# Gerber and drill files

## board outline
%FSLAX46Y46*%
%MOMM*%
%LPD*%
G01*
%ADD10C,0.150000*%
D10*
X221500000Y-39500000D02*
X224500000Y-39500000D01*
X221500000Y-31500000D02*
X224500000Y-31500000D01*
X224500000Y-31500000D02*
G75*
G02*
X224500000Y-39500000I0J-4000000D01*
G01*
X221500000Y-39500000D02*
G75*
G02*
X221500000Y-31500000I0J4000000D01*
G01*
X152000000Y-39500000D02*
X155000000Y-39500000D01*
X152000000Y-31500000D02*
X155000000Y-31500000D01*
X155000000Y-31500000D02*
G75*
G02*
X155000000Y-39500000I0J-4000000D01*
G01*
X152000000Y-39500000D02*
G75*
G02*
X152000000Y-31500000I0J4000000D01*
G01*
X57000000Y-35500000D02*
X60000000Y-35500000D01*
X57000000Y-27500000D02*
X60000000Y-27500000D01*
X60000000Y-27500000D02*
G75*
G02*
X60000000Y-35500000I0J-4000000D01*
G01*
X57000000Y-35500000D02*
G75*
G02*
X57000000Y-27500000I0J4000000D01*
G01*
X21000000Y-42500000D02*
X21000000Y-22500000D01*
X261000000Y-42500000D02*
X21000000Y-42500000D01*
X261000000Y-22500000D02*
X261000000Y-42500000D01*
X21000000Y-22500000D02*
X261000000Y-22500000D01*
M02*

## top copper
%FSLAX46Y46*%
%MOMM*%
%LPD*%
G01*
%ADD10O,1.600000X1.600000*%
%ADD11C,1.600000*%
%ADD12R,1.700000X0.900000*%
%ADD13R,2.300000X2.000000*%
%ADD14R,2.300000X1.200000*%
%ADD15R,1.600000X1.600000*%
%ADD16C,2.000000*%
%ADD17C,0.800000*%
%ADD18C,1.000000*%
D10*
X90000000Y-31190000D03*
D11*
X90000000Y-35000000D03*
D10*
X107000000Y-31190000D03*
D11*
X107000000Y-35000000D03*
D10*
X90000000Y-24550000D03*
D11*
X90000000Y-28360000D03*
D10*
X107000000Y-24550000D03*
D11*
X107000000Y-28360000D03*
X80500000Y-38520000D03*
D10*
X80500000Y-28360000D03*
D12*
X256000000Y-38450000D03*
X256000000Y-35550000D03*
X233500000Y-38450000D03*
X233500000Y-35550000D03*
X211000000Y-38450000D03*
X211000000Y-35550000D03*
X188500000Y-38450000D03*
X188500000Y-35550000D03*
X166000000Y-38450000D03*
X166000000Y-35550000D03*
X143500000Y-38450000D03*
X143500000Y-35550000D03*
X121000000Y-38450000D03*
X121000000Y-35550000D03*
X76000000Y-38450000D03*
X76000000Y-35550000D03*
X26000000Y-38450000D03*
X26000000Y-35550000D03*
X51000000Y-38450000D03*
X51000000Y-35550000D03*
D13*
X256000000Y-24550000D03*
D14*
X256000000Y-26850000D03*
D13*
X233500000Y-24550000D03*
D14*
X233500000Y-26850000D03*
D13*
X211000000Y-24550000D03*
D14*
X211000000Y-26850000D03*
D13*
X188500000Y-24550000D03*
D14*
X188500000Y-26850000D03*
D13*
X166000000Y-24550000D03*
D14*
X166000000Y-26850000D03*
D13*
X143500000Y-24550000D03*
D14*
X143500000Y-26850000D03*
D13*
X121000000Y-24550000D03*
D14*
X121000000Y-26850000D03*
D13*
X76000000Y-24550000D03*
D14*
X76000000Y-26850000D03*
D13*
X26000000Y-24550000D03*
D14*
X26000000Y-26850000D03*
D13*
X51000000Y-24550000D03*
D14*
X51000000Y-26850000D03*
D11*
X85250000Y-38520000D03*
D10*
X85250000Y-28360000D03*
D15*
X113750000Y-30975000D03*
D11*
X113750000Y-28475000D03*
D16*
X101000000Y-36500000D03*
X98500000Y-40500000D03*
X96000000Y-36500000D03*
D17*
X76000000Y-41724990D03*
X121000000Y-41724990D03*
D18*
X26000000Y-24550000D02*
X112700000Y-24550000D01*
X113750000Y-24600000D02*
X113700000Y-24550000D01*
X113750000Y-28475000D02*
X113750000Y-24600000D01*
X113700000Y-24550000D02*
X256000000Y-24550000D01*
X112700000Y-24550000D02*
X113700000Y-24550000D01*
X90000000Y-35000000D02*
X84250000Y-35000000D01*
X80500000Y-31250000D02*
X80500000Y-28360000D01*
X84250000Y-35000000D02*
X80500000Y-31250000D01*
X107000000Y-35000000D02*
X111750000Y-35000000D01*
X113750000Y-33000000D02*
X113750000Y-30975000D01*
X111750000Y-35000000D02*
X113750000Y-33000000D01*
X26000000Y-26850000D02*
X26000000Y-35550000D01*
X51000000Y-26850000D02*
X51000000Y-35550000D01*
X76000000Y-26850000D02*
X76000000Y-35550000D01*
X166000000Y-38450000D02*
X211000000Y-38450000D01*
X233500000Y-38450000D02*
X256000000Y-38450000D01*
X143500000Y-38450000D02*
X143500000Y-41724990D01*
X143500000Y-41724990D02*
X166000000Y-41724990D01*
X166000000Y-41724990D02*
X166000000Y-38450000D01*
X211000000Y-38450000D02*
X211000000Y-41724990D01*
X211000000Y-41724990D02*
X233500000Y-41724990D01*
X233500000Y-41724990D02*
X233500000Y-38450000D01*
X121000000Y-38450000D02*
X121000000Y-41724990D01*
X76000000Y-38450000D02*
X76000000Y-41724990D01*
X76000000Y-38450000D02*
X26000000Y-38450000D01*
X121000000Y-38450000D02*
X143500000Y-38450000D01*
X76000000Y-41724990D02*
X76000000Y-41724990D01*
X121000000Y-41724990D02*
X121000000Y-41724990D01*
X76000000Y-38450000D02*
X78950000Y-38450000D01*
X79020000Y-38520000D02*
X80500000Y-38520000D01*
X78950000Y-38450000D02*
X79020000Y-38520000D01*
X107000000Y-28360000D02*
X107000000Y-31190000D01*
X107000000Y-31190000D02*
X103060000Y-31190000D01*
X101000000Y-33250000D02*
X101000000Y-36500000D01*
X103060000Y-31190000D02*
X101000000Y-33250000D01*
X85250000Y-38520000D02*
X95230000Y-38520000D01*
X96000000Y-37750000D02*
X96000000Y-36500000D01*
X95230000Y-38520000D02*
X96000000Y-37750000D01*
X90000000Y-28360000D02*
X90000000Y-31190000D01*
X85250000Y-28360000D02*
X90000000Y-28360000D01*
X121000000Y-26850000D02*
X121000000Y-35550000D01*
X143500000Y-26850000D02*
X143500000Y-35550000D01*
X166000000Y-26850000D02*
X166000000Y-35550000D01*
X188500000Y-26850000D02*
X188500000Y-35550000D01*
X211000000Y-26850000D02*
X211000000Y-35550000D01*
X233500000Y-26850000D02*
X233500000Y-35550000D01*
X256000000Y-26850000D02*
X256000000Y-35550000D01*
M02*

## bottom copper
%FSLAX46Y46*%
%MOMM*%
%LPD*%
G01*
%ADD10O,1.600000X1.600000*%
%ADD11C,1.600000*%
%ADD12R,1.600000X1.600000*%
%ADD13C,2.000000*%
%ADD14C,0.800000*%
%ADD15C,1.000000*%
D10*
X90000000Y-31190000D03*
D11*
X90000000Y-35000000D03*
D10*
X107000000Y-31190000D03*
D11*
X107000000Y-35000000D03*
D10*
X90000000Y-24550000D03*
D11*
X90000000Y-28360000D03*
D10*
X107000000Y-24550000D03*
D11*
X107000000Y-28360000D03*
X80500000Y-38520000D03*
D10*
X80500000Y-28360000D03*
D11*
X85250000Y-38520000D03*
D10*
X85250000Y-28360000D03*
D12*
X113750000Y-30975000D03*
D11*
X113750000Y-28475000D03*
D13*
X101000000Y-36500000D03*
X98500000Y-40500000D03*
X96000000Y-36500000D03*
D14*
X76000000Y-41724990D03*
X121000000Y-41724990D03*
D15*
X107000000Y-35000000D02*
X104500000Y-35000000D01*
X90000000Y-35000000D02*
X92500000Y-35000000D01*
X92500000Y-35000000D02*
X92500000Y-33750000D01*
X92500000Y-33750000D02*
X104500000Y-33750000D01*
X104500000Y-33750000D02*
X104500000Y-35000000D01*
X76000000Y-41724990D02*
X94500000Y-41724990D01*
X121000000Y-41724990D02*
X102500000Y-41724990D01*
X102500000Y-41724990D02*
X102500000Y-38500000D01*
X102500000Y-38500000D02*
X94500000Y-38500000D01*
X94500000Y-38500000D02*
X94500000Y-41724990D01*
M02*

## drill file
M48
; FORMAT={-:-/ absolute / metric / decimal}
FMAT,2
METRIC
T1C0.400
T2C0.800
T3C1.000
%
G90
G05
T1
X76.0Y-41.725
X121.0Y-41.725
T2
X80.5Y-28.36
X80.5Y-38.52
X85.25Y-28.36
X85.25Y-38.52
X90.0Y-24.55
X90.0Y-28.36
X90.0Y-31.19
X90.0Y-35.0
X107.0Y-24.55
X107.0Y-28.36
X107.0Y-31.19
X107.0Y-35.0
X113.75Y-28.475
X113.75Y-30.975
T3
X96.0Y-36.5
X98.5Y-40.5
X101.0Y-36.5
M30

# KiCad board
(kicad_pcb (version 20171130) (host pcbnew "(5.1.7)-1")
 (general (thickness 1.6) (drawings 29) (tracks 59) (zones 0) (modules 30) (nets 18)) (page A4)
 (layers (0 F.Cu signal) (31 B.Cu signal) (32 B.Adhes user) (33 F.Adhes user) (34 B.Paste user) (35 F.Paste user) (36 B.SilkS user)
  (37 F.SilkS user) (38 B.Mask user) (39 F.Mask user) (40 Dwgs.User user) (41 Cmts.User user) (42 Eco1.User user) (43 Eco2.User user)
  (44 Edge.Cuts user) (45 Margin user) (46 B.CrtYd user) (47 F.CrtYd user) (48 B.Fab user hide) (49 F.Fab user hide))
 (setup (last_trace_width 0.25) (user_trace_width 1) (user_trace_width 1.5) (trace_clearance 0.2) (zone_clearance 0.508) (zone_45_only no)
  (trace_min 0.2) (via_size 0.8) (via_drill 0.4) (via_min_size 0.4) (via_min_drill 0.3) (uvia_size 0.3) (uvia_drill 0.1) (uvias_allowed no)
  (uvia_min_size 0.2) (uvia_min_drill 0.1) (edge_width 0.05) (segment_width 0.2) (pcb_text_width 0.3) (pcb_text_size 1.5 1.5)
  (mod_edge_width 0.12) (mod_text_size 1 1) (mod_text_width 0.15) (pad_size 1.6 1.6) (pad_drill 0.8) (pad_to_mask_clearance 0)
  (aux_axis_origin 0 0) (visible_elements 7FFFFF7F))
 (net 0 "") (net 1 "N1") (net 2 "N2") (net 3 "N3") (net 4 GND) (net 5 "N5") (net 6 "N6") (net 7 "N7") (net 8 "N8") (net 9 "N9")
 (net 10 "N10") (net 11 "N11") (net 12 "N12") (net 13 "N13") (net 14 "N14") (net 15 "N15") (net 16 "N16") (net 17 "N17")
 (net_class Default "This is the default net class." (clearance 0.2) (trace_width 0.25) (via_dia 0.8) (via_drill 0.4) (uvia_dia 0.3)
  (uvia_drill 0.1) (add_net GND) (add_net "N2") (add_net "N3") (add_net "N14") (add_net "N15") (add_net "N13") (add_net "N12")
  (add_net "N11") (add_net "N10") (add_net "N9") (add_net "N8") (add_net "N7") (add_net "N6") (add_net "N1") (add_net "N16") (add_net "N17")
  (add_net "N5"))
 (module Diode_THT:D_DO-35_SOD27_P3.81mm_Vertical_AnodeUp (layer F.Cu) (at 90 35 90)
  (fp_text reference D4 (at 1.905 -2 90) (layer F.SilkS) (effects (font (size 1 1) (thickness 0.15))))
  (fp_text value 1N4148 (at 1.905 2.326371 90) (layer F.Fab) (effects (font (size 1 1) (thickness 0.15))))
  (pad 2 thru_hole oval (at 3.81 0 90) (size 1.6 1.6) (drill 0.8) (layers *.Cu *.Mask) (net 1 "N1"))
  (pad 1 thru_hole circle (at 0 0 90) (size 1.6 1.6) (drill 0.8) (layers *.Cu *.Mask) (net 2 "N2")))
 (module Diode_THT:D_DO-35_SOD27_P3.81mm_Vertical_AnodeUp (layer F.Cu) (at 107 35 90)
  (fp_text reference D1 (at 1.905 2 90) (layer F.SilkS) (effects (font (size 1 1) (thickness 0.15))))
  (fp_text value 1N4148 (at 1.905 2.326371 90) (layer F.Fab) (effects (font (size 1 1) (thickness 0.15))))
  (pad 2 thru_hole oval (at 3.81 0 90) (size 1.6 1.6) (drill 0.8) (layers *.Cu *.Mask) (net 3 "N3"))
  (pad 1 thru_hole circle (at 0 0 90) (size 1.6 1.6) (drill 0.8) (layers *.Cu *.Mask) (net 2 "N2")))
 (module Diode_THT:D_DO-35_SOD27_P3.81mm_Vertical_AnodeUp (layer F.Cu) (at 90 28.36 90)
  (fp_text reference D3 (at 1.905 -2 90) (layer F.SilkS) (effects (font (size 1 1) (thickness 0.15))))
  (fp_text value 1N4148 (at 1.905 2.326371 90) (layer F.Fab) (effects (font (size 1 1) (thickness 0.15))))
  (pad 2 thru_hole oval (at 3.81 0 90) (size 1.6 1.6) (drill 0.8) (layers *.Cu *.Mask) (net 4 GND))
  (pad 1 thru_hole circle (at 0 0 90) (size 1.6 1.6) (drill 0.8) (layers *.Cu *.Mask) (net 1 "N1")))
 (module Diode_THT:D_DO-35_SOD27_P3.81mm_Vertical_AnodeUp (layer F.Cu) (at 107 28.36 90)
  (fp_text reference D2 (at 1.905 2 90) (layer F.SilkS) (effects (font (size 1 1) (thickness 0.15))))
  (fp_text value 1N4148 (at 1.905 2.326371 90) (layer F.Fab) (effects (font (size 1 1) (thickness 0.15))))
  (pad 2 thru_hole oval (at 3.81 0 90) (size 1.6 1.6) (drill 0.8) (layers *.Cu *.Mask) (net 4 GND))
  (pad 1 thru_hole circle (at 0 0 90) (size 1.6 1.6) (drill 0.8) (layers *.Cu *.Mask) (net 3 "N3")))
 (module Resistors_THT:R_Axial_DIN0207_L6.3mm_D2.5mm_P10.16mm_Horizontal (layer F.Cu) (at 80.5 38.52 90)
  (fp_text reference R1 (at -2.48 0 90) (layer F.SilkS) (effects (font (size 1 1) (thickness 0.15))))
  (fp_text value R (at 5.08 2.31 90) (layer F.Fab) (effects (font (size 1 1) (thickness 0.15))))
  (pad 1 thru_hole circle (at 0 0 90) (size 1.6 1.6) (drill 0.8) (layers *.Cu *.Mask) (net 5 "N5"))
  (pad 2 thru_hole oval (at 10.16 0 90) (size 1.6 1.6) (drill 0.8) (layers *.Cu *.Mask) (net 2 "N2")))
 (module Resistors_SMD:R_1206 (layer F.Cu) (at 256 37 90)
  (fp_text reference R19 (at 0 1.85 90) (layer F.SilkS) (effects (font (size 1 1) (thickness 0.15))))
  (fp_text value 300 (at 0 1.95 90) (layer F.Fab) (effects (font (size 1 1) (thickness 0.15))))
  (pad 1 smd rect (at -1.45 0 90) (size 0.9 1.7) (layers F.Cu F.Paste F.Mask) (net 5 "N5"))
  (pad 2 smd rect (at 1.45 0 90) (size 0.9 1.7) (layers F.Cu F.Paste F.Mask) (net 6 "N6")))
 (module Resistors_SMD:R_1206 (layer F.Cu) (at 233.5 37 90)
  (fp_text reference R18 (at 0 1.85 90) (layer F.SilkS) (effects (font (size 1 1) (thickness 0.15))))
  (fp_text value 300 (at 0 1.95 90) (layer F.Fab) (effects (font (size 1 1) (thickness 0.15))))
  (pad 1 smd rect (at -1.45 0 90) (size 0.9 1.7) (layers F.Cu F.Paste F.Mask) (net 5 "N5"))
  (pad 2 smd rect (at 1.45 0 90) (size 0.9 1.7) (layers F.Cu F.Paste F.Mask) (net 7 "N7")))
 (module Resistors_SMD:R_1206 (layer F.Cu) (at 211 37 90)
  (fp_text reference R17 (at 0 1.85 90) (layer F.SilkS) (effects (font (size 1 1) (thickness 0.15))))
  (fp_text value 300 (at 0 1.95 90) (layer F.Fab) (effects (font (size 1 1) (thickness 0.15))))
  (pad 1 smd rect (at -1.45 0 90) (size 0.9 1.7) (layers F.Cu F.Paste F.Mask) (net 5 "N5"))
  (pad 2 smd rect (at 1.45 0 90) (size 0.9 1.7) (layers F.Cu F.Paste F.Mask) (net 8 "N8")))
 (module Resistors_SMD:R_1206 (layer F.Cu) (at 188.5 37 90)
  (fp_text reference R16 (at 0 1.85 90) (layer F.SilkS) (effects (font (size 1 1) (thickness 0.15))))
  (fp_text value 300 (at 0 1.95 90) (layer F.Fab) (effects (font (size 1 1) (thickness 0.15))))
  (pad 1 smd rect (at -1.45 0 90) (size 0.9 1.7) (layers F.Cu F.Paste F.Mask) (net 5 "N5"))
  (pad 2 smd rect (at 1.45 0 90) (size 0.9 1.7) (layers F.Cu F.Paste F.Mask) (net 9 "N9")))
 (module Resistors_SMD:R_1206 (layer F.Cu) (at 166 37 90)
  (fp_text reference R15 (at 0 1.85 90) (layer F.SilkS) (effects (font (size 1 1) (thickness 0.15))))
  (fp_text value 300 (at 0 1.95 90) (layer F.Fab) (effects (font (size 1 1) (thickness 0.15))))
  (pad 1 smd rect (at -1.45 0 90) (size 0.9 1.7) (layers F.Cu F.Paste F.Mask) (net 5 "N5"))
  (pad 2 smd rect (at 1.45 0 90) (size 0.9 1.7) (layers F.Cu F.Paste F.Mask) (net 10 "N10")))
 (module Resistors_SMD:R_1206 (layer F.Cu) (at 143.5 37 90)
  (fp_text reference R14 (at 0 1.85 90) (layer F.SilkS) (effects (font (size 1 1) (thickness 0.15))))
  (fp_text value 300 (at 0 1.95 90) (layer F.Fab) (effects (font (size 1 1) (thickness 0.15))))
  (pad 1 smd rect (at -1.45 0 90) (size 0.9 1.7) (layers F.Cu F.Paste F.Mask) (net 5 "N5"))
  (pad 2 smd rect (at 1.45 0 90) (size 0.9 1.7) (layers F.Cu F.Paste F.Mask) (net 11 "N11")))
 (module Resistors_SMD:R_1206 (layer F.Cu) (at 121 37 90)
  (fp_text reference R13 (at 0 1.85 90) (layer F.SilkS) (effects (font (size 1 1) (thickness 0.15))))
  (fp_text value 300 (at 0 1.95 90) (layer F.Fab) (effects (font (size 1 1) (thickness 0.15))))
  (pad 1 smd rect (at -1.45 0 90) (size 0.9 1.7) (layers F.Cu F.Paste F.Mask) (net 5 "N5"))
  (pad 2 smd rect (at 1.45 0 90) (size 0.9 1.7) (layers F.Cu F.Paste F.Mask) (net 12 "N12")))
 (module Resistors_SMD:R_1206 (layer F.Cu) (at 76 37 90)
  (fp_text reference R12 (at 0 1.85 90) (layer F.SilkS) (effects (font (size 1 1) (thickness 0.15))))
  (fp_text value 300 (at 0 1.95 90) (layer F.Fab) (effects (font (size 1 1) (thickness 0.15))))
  (pad 1 smd rect (at -1.45 0 90) (size 0.9 1.7) (layers F.Cu F.Paste F.Mask) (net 5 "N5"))
  (pad 2 smd rect (at 1.45 0 90) (size 0.9 1.7) (layers F.Cu F.Paste F.Mask) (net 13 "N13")))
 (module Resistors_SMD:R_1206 (layer F.Cu) (at 26 37 90)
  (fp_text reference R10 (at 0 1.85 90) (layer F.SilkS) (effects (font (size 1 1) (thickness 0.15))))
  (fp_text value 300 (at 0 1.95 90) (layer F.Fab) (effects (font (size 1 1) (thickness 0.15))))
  (pad 1 smd rect (at -1.45 0 90) (size 0.9 1.7) (layers F.Cu F.Paste F.Mask) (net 5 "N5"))
  (pad 2 smd rect (at 1.45 0 90) (size 0.9 1.7) (layers F.Cu F.Paste F.Mask) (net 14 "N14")))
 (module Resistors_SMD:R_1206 (layer F.Cu) (at 51 37 90)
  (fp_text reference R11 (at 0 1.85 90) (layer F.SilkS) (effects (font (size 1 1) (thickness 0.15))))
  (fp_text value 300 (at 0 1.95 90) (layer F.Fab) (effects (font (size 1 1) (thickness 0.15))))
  (pad 1 smd rect (at -1.45 0 90) (size 0.9 1.7) (layers F.Cu F.Paste F.Mask) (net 5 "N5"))
  (pad 2 smd rect (at 1.45 0 90) (size 0.9 1.7) (layers F.Cu F.Paste F.Mask) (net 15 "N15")))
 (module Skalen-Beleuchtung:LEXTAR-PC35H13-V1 (layer F.Cu) (at 256 25.5 90)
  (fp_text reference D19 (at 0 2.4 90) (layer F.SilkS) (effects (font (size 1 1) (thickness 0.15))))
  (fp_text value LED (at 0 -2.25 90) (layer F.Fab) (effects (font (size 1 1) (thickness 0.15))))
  (pad 1 smd rect (at 0.95 0 90) (size 2 2.3) (layers F.Cu F.Paste F.Mask) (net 4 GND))
  (pad 2 smd rect (at -1.35 0 90) (size 1.2 2.3) (layers F.Cu F.Paste F.Mask) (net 6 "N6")))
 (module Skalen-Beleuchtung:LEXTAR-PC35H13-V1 (layer F.Cu) (at 233.5 25.5 90)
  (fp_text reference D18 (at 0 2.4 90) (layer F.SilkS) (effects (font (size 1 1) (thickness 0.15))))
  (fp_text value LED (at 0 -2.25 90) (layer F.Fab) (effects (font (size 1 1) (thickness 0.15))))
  (pad 1 smd rect (at 0.95 0 90) (size 2 2.3) (layers F.Cu F.Paste F.Mask) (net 4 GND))
  (pad 2 smd rect (at -1.35 0 90) (size 1.2 2.3) (layers F.Cu F.Paste F.Mask) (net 7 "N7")))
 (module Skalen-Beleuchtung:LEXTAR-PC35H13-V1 (layer F.Cu) (at 211 25.5 90)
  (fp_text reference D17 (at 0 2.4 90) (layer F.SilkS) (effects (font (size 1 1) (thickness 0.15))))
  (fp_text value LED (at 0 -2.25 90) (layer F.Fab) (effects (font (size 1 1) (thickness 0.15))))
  (pad 1 smd rect (at 0.95 0 90) (size 2 2.3) (layers F.Cu F.Paste F.Mask) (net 4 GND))
  (pad 2 smd rect (at -1.35 0 90) (size 1.2 2.3) (layers F.Cu F.Paste F.Mask) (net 8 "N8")))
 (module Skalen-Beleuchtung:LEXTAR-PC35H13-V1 (layer F.Cu) (at 188.5 25.5 90)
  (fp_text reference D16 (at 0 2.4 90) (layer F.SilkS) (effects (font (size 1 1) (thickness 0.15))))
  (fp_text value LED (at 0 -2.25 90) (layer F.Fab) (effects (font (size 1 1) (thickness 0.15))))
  (pad 1 smd rect (at 0.95 0 90) (size 2 2.3) (layers F.Cu F.Paste F.Mask) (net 4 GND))
  (pad 2 smd rect (at -1.35 0 90) (size 1.2 2.3) (layers F.Cu F.Paste F.Mask) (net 9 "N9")))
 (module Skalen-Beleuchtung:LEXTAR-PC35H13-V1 (layer F.Cu) (at 166 25.5 90)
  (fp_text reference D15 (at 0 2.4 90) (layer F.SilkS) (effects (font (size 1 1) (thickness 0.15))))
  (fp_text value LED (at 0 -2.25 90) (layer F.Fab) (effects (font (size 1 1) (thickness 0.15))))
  (pad 1 smd rect (at 0.95 0 90) (size 2 2.3) (layers F.Cu F.Paste F.Mask) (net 4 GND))
  (pad 2 smd rect (at -1.35 0 90) (size 1.2 2.3) (layers F.Cu F.Paste F.Mask) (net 10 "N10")))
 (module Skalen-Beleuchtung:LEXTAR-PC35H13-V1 (layer F.Cu) (at 143.5 25.5 90)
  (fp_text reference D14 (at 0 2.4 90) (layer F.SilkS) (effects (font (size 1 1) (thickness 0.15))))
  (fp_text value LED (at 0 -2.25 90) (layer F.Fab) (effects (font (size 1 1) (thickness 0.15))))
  (pad 1 smd rect (at 0.95 0 90) (size 2 2.3) (layers F.Cu F.Paste F.Mask) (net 4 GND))
  (pad 2 smd rect (at -1.35 0 90) (size 1.2 2.3) (layers F.Cu F.Paste F.Mask) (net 11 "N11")))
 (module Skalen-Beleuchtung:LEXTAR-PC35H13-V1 (layer F.Cu) (at 121 25.5 90)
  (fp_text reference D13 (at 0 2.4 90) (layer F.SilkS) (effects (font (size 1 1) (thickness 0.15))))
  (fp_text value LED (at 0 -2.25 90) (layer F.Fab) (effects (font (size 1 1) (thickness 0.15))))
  (pad 1 smd rect (at 0.95 0 90) (size 2 2.3) (layers F.Cu F.Paste F.Mask) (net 4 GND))
  (pad 2 smd rect (at -1.35 0 90) (size 1.2 2.3) (layers F.Cu F.Paste F.Mask) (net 12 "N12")))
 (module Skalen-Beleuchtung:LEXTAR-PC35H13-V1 (layer F.Cu) (at 76 25.5 90)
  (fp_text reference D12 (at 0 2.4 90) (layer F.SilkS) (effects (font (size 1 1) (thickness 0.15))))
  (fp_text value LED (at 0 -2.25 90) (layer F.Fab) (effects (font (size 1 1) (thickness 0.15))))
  (pad 1 smd rect (at 0.95 0 90) (size 2 2.3) (layers F.Cu F.Paste F.Mask) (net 4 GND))
  (pad 2 smd rect (at -1.35 0 90) (size 1.2 2.3) (layers F.Cu F.Paste F.Mask) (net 13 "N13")))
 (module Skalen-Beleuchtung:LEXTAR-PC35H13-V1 (layer F.Cu) (at 26 25.5 90)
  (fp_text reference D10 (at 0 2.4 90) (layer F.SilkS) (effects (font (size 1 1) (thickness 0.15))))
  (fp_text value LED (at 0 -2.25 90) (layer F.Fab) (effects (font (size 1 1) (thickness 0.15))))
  (pad 1 smd rect (at 0.95 0 90) (size 2 2.3) (layers F.Cu F.Paste F.Mask) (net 4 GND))
  (pad 2 smd rect (at -1.35 0 90) (size 1.2 2.3) (layers F.Cu F.Paste F.Mask) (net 14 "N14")))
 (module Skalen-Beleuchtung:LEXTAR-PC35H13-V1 (layer F.Cu) (at 51 25.5 90)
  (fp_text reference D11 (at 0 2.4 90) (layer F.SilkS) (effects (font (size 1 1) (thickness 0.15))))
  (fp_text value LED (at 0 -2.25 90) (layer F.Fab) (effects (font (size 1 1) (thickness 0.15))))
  (pad 1 smd rect (at 0.95 0 90) (size 2 2.3) (layers F.Cu F.Paste F.Mask) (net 4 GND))
  (pad 2 smd rect (at -1.35 0 90) (size 1.2 2.3) (layers F.Cu F.Paste F.Mask) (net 15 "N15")))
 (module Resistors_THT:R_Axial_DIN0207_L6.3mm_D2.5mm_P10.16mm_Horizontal (layer F.Cu) (at 85.25 38.52 90)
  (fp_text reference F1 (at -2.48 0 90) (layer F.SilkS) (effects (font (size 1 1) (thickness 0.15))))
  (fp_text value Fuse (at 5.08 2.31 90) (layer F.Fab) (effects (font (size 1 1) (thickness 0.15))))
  (pad 1 thru_hole circle (at 0 0 90) (size 1.6 1.6) (drill 0.8) (layers *.Cu *.Mask) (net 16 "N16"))
  (pad 2 thru_hole oval (at 10.16 0 90) (size 1.6 1.6) (drill 0.8) (layers *.Cu *.Mask) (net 1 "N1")))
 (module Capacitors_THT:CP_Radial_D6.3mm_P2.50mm (layer F.Cu) (at 113.75 30.975 90)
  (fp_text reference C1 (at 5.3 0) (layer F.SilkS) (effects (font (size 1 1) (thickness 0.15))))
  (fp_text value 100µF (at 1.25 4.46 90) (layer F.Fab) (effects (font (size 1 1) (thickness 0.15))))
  (pad 1 thru_hole rect (at 0 0 90) (size 1.6 1.6) (drill 0.8) (layers *.Cu *.Mask) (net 2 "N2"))
  (pad 2 thru_hole circle (at 2.5 0 90) (size 1.6 1.6) (drill 0.8) (layers *.Cu *.Mask) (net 4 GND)))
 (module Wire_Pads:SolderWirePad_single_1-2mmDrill (layer F.Cu) (at 101 36.5)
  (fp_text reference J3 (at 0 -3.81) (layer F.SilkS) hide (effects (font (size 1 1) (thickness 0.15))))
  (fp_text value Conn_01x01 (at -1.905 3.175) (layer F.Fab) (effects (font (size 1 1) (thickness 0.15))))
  (pad 1 thru_hole circle (at 0 0) (size 2 2) (drill 1) (layers *.Cu *.Mask) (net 3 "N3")))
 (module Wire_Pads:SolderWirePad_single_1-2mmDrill (layer F.Cu) (at 98.5 40.5)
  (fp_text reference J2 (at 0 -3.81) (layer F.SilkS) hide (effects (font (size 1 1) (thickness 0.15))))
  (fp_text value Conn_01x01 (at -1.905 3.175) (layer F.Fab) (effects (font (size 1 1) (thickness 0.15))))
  (pad 1 thru_hole circle (at 0 0) (size 2 2) (drill 1) (layers *.Cu *.Mask) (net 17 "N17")))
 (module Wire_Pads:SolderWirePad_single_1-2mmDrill (layer F.Cu) (at 96 36.5)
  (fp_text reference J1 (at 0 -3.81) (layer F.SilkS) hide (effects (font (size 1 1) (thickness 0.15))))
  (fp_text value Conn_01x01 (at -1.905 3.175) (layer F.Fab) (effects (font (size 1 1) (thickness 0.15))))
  (pad 1 thru_hole circle (at 0 0) (size 2 2) (drill 1) (layers *.Cu *.Mask) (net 16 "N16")))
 (gr_line (start 221.5 39.5) (end 224.5 39.5) (layer Edge.Cuts) (width 0.15))
 (gr_line (start 221.5 31.5) (end 224.5 31.5) (layer Edge.Cuts) (width 0.15))
 (gr_arc (start 224.5 35.5) (end 224.5 39.5) (angle -180) (layer Edge.Cuts) (width 0.15))
 (gr_arc (start 221.5 35.5) (end 221.5 31.5) (angle -180) (layer Edge.Cuts) (width 0.15))
 (gr_line (start 152 39.5) (end 155 39.5) (layer Edge.Cuts) (width 0.15))
 (gr_line (start 152 31.5) (end 155 31.5) (layer Edge.Cuts) (width 0.15))
 (gr_arc (start 155 35.5) (end 155 39.5) (angle -180) (layer Edge.Cuts) (width 0.15))
 (gr_arc (start 152 35.5) (end 152 31.5) (angle -180) (layer Edge.Cuts) (width 0.15))
 (gr_line (start 57 35.5) (end 60 35.5) (layer Edge.Cuts) (width 0.15))
 (gr_line (start 57 27.5) (end 60 27.5) (layer Edge.Cuts) (width 0.15))
 (gr_arc (start 60 31.5) (end 60 35.5) (angle -180) (layer Edge.Cuts) (width 0.15))
 (gr_arc (start 57 31.5) (end 57 27.5) (angle -180) (layer Edge.Cuts) (width 0.15))
 (gr_line (start 21 42.5) (end 21 22.5) (layer Edge.Cuts) (width 0.15))
 (gr_line (start 261 42.5) (end 21 42.5) (layer Edge.Cuts) (width 0.15))
 (gr_line (start 261 22.5) (end 261 42.5) (layer Edge.Cuts) (width 0.15))
 (gr_line (start 21 22.5) (end 261 22.5) (layer Edge.Cuts) (width 0.15))
 (segment (start 26 24.55) (end 112.7 24.55) (width 1) (layer F.Cu) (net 4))
 (segment (start 113.75 24.6) (end 113.7 24.55) (width 1) (layer F.Cu) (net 4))
 (segment (start 113.75 28.475) (end 113.75 24.6) (width 1) (layer F.Cu) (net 4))
 (segment (start 113.7 24.55) (end 256 24.55) (width 1) (layer F.Cu) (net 4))
 (segment (start 112.7 24.55) (end 113.7 24.55) (width 1) (layer F.Cu) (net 4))
 (segment (start 107 35) (end 104.5 35) (width 1) (layer B.Cu) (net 2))
 (segment (start 90 35) (end 92.5 35) (width 1) (layer B.Cu) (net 2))
 (segment (start 92.5 35) (end 92.5 33.75) (width 1) (layer B.Cu) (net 2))
 (segment (start 92.5 33.75) (end 104.5 33.75) (width 1) (layer B.Cu) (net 2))
 (segment (start 104.5 33.75) (end 104.5 35) (width 1) (layer B.Cu) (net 2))
 (segment (start 90 35) (end 84.25 35) (width 1) (layer F.Cu) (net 2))
 (segment (start 80.5 31.25) (end 80.5 28.36) (width 1) (layer F.Cu) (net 2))
 (segment (start 84.25 35) (end 80.5 31.25) (width 1) (layer F.Cu) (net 2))
 (segment (start 107 35) (end 111.75 35) (width 1) (layer F.Cu) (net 2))
 (segment (start 113.75 33) (end 113.75 30.975) (width 1) (layer F.Cu) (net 2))
 (segment (start 111.75 35) (end 113.75 33) (width 1) (layer F.Cu) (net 2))
 (segment (start 26 26.85) (end 26 35.55) (width 1) (layer F.Cu) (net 14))
 (segment (start 51 26.85) (end 51 35.55) (width 1) (layer F.Cu) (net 15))
 (segment (start 76 26.85) (end 76 35.55) (width 1) (layer F.Cu) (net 13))
 (segment (start 166 38.45) (end 211 38.45) (width 1) (layer F.Cu) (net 5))
 (segment (start 233.5 38.45) (end 256 38.45) (width 1) (layer F.Cu) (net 5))
 (segment (start 143.5 38.45) (end 143.5 41.72499) (width 1) (layer F.Cu) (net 5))
 (segment (start 143.5 41.72499) (end 166 41.72499) (width 1) (layer F.Cu) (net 5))
 (segment (start 166 41.72499) (end 166 38.45) (width 1) (layer F.Cu) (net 5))
 (segment (start 211 38.45) (end 211 41.72499) (width 1) (layer F.Cu) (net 5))
 (segment (start 211 41.72499) (end 233.5 41.72499) (width 1) (layer F.Cu) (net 5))
 (segment (start 233.5 41.72499) (end 233.5 38.45) (width 1) (layer F.Cu) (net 5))
 (segment (start 121 38.45) (end 121 41.72499) (width 1) (layer F.Cu) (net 5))
 (segment (start 76 38.45) (end 76 41.72499) (width 1) (layer F.Cu) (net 5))
 (segment (start 76 38.45) (end 26 38.45) (width 1) (layer F.Cu) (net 5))
 (segment (start 121 38.45) (end 143.5 38.45) (width 1) (layer F.Cu) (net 5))
 (segment (start 76 41.72499) (end 76 41.72499) (width 1) (layer F.Cu) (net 5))
 (via (at 76 41.72499) (size 0.8) (drill 0.4) (layers F.Cu B.Cu) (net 5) (status 1000000))
 (segment (start 121 41.72499) (end 121 41.72499) (width 1) (layer F.Cu) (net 5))
 (via (at 121 41.72499) (size 0.8) (drill 0.4) (layers F.Cu B.Cu) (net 5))
 (segment (start 76 41.72499) (end 94.5 41.72499) (width 1) (layer B.Cu) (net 5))
 (segment (start 121 41.72499) (end 102.5 41.72499) (width 1) (layer B.Cu) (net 5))
 (segment (start 102.5 41.72499) (end 102.5 38.5) (width 1) (layer B.Cu) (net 5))
 (segment (start 102.5 38.5) (end 94.5 38.5) (width 1) (layer B.Cu) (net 5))
 (segment (start 94.5 38.5) (end 94.5 41.72499) (width 1) (layer B.Cu) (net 5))
 (segment (start 76 38.45) (end 78.95 38.45) (width 1) (layer F.Cu) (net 5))
 (segment (start 79.02 38.52) (end 80.5 38.52) (width 1) (layer F.Cu) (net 5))
 (segment (start 78.95 38.45) (end 79.02 38.52) (width 1) (layer F.Cu) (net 5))
 (segment (start 107 28.36) (end 107 31.19) (width 1) (layer F.Cu) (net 3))
 (segment (start 107 31.19) (end 103.06 31.19) (width 1) (layer F.Cu) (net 3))
 (segment (start 101 33.25) (end 101 36.5) (width 1) (layer F.Cu) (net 3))
 (segment (start 103.06 31.19) (end 101 33.25) (width 1) (layer F.Cu) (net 3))
 (segment (start 85.25 38.52) (end 95.23 38.52) (width 1) (layer F.Cu) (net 16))
 (segment (start 96 37.75) (end 96 36.5) (width 1) (layer F.Cu) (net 16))
 (segment (start 95.23 38.52) (end 96 37.75) (width 1) (layer F.Cu) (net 16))
 (segment (start 90 28.36) (end 90 31.19) (width 1) (layer F.Cu) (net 1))
 (segment (start 85.25 28.36) (end 90 28.36) (width 1) (layer F.Cu) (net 1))
 (segment (start 121 26.85) (end 121 35.55) (width 1) (layer F.Cu) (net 12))
 (segment (start 143.5 26.85) (end 143.5 35.55) (width 1) (layer F.Cu) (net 11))
 (segment (start 166 26.85) (end 166 35.55) (width 1) (layer F.Cu) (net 10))
 (segment (start 188.5 26.85) (end 188.5 35.55) (width 1) (layer F.Cu) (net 9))
 (segment (start 211 26.85) (end 211 35.55) (width 1) (layer F.Cu) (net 8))
 (segment (start 233.5 26.85) (end 233.5 35.55) (width 1) (layer F.Cu) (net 7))
 (segment (start 256 26.85) (end 256 35.55) (width 1) (layer F.Cu) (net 6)))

